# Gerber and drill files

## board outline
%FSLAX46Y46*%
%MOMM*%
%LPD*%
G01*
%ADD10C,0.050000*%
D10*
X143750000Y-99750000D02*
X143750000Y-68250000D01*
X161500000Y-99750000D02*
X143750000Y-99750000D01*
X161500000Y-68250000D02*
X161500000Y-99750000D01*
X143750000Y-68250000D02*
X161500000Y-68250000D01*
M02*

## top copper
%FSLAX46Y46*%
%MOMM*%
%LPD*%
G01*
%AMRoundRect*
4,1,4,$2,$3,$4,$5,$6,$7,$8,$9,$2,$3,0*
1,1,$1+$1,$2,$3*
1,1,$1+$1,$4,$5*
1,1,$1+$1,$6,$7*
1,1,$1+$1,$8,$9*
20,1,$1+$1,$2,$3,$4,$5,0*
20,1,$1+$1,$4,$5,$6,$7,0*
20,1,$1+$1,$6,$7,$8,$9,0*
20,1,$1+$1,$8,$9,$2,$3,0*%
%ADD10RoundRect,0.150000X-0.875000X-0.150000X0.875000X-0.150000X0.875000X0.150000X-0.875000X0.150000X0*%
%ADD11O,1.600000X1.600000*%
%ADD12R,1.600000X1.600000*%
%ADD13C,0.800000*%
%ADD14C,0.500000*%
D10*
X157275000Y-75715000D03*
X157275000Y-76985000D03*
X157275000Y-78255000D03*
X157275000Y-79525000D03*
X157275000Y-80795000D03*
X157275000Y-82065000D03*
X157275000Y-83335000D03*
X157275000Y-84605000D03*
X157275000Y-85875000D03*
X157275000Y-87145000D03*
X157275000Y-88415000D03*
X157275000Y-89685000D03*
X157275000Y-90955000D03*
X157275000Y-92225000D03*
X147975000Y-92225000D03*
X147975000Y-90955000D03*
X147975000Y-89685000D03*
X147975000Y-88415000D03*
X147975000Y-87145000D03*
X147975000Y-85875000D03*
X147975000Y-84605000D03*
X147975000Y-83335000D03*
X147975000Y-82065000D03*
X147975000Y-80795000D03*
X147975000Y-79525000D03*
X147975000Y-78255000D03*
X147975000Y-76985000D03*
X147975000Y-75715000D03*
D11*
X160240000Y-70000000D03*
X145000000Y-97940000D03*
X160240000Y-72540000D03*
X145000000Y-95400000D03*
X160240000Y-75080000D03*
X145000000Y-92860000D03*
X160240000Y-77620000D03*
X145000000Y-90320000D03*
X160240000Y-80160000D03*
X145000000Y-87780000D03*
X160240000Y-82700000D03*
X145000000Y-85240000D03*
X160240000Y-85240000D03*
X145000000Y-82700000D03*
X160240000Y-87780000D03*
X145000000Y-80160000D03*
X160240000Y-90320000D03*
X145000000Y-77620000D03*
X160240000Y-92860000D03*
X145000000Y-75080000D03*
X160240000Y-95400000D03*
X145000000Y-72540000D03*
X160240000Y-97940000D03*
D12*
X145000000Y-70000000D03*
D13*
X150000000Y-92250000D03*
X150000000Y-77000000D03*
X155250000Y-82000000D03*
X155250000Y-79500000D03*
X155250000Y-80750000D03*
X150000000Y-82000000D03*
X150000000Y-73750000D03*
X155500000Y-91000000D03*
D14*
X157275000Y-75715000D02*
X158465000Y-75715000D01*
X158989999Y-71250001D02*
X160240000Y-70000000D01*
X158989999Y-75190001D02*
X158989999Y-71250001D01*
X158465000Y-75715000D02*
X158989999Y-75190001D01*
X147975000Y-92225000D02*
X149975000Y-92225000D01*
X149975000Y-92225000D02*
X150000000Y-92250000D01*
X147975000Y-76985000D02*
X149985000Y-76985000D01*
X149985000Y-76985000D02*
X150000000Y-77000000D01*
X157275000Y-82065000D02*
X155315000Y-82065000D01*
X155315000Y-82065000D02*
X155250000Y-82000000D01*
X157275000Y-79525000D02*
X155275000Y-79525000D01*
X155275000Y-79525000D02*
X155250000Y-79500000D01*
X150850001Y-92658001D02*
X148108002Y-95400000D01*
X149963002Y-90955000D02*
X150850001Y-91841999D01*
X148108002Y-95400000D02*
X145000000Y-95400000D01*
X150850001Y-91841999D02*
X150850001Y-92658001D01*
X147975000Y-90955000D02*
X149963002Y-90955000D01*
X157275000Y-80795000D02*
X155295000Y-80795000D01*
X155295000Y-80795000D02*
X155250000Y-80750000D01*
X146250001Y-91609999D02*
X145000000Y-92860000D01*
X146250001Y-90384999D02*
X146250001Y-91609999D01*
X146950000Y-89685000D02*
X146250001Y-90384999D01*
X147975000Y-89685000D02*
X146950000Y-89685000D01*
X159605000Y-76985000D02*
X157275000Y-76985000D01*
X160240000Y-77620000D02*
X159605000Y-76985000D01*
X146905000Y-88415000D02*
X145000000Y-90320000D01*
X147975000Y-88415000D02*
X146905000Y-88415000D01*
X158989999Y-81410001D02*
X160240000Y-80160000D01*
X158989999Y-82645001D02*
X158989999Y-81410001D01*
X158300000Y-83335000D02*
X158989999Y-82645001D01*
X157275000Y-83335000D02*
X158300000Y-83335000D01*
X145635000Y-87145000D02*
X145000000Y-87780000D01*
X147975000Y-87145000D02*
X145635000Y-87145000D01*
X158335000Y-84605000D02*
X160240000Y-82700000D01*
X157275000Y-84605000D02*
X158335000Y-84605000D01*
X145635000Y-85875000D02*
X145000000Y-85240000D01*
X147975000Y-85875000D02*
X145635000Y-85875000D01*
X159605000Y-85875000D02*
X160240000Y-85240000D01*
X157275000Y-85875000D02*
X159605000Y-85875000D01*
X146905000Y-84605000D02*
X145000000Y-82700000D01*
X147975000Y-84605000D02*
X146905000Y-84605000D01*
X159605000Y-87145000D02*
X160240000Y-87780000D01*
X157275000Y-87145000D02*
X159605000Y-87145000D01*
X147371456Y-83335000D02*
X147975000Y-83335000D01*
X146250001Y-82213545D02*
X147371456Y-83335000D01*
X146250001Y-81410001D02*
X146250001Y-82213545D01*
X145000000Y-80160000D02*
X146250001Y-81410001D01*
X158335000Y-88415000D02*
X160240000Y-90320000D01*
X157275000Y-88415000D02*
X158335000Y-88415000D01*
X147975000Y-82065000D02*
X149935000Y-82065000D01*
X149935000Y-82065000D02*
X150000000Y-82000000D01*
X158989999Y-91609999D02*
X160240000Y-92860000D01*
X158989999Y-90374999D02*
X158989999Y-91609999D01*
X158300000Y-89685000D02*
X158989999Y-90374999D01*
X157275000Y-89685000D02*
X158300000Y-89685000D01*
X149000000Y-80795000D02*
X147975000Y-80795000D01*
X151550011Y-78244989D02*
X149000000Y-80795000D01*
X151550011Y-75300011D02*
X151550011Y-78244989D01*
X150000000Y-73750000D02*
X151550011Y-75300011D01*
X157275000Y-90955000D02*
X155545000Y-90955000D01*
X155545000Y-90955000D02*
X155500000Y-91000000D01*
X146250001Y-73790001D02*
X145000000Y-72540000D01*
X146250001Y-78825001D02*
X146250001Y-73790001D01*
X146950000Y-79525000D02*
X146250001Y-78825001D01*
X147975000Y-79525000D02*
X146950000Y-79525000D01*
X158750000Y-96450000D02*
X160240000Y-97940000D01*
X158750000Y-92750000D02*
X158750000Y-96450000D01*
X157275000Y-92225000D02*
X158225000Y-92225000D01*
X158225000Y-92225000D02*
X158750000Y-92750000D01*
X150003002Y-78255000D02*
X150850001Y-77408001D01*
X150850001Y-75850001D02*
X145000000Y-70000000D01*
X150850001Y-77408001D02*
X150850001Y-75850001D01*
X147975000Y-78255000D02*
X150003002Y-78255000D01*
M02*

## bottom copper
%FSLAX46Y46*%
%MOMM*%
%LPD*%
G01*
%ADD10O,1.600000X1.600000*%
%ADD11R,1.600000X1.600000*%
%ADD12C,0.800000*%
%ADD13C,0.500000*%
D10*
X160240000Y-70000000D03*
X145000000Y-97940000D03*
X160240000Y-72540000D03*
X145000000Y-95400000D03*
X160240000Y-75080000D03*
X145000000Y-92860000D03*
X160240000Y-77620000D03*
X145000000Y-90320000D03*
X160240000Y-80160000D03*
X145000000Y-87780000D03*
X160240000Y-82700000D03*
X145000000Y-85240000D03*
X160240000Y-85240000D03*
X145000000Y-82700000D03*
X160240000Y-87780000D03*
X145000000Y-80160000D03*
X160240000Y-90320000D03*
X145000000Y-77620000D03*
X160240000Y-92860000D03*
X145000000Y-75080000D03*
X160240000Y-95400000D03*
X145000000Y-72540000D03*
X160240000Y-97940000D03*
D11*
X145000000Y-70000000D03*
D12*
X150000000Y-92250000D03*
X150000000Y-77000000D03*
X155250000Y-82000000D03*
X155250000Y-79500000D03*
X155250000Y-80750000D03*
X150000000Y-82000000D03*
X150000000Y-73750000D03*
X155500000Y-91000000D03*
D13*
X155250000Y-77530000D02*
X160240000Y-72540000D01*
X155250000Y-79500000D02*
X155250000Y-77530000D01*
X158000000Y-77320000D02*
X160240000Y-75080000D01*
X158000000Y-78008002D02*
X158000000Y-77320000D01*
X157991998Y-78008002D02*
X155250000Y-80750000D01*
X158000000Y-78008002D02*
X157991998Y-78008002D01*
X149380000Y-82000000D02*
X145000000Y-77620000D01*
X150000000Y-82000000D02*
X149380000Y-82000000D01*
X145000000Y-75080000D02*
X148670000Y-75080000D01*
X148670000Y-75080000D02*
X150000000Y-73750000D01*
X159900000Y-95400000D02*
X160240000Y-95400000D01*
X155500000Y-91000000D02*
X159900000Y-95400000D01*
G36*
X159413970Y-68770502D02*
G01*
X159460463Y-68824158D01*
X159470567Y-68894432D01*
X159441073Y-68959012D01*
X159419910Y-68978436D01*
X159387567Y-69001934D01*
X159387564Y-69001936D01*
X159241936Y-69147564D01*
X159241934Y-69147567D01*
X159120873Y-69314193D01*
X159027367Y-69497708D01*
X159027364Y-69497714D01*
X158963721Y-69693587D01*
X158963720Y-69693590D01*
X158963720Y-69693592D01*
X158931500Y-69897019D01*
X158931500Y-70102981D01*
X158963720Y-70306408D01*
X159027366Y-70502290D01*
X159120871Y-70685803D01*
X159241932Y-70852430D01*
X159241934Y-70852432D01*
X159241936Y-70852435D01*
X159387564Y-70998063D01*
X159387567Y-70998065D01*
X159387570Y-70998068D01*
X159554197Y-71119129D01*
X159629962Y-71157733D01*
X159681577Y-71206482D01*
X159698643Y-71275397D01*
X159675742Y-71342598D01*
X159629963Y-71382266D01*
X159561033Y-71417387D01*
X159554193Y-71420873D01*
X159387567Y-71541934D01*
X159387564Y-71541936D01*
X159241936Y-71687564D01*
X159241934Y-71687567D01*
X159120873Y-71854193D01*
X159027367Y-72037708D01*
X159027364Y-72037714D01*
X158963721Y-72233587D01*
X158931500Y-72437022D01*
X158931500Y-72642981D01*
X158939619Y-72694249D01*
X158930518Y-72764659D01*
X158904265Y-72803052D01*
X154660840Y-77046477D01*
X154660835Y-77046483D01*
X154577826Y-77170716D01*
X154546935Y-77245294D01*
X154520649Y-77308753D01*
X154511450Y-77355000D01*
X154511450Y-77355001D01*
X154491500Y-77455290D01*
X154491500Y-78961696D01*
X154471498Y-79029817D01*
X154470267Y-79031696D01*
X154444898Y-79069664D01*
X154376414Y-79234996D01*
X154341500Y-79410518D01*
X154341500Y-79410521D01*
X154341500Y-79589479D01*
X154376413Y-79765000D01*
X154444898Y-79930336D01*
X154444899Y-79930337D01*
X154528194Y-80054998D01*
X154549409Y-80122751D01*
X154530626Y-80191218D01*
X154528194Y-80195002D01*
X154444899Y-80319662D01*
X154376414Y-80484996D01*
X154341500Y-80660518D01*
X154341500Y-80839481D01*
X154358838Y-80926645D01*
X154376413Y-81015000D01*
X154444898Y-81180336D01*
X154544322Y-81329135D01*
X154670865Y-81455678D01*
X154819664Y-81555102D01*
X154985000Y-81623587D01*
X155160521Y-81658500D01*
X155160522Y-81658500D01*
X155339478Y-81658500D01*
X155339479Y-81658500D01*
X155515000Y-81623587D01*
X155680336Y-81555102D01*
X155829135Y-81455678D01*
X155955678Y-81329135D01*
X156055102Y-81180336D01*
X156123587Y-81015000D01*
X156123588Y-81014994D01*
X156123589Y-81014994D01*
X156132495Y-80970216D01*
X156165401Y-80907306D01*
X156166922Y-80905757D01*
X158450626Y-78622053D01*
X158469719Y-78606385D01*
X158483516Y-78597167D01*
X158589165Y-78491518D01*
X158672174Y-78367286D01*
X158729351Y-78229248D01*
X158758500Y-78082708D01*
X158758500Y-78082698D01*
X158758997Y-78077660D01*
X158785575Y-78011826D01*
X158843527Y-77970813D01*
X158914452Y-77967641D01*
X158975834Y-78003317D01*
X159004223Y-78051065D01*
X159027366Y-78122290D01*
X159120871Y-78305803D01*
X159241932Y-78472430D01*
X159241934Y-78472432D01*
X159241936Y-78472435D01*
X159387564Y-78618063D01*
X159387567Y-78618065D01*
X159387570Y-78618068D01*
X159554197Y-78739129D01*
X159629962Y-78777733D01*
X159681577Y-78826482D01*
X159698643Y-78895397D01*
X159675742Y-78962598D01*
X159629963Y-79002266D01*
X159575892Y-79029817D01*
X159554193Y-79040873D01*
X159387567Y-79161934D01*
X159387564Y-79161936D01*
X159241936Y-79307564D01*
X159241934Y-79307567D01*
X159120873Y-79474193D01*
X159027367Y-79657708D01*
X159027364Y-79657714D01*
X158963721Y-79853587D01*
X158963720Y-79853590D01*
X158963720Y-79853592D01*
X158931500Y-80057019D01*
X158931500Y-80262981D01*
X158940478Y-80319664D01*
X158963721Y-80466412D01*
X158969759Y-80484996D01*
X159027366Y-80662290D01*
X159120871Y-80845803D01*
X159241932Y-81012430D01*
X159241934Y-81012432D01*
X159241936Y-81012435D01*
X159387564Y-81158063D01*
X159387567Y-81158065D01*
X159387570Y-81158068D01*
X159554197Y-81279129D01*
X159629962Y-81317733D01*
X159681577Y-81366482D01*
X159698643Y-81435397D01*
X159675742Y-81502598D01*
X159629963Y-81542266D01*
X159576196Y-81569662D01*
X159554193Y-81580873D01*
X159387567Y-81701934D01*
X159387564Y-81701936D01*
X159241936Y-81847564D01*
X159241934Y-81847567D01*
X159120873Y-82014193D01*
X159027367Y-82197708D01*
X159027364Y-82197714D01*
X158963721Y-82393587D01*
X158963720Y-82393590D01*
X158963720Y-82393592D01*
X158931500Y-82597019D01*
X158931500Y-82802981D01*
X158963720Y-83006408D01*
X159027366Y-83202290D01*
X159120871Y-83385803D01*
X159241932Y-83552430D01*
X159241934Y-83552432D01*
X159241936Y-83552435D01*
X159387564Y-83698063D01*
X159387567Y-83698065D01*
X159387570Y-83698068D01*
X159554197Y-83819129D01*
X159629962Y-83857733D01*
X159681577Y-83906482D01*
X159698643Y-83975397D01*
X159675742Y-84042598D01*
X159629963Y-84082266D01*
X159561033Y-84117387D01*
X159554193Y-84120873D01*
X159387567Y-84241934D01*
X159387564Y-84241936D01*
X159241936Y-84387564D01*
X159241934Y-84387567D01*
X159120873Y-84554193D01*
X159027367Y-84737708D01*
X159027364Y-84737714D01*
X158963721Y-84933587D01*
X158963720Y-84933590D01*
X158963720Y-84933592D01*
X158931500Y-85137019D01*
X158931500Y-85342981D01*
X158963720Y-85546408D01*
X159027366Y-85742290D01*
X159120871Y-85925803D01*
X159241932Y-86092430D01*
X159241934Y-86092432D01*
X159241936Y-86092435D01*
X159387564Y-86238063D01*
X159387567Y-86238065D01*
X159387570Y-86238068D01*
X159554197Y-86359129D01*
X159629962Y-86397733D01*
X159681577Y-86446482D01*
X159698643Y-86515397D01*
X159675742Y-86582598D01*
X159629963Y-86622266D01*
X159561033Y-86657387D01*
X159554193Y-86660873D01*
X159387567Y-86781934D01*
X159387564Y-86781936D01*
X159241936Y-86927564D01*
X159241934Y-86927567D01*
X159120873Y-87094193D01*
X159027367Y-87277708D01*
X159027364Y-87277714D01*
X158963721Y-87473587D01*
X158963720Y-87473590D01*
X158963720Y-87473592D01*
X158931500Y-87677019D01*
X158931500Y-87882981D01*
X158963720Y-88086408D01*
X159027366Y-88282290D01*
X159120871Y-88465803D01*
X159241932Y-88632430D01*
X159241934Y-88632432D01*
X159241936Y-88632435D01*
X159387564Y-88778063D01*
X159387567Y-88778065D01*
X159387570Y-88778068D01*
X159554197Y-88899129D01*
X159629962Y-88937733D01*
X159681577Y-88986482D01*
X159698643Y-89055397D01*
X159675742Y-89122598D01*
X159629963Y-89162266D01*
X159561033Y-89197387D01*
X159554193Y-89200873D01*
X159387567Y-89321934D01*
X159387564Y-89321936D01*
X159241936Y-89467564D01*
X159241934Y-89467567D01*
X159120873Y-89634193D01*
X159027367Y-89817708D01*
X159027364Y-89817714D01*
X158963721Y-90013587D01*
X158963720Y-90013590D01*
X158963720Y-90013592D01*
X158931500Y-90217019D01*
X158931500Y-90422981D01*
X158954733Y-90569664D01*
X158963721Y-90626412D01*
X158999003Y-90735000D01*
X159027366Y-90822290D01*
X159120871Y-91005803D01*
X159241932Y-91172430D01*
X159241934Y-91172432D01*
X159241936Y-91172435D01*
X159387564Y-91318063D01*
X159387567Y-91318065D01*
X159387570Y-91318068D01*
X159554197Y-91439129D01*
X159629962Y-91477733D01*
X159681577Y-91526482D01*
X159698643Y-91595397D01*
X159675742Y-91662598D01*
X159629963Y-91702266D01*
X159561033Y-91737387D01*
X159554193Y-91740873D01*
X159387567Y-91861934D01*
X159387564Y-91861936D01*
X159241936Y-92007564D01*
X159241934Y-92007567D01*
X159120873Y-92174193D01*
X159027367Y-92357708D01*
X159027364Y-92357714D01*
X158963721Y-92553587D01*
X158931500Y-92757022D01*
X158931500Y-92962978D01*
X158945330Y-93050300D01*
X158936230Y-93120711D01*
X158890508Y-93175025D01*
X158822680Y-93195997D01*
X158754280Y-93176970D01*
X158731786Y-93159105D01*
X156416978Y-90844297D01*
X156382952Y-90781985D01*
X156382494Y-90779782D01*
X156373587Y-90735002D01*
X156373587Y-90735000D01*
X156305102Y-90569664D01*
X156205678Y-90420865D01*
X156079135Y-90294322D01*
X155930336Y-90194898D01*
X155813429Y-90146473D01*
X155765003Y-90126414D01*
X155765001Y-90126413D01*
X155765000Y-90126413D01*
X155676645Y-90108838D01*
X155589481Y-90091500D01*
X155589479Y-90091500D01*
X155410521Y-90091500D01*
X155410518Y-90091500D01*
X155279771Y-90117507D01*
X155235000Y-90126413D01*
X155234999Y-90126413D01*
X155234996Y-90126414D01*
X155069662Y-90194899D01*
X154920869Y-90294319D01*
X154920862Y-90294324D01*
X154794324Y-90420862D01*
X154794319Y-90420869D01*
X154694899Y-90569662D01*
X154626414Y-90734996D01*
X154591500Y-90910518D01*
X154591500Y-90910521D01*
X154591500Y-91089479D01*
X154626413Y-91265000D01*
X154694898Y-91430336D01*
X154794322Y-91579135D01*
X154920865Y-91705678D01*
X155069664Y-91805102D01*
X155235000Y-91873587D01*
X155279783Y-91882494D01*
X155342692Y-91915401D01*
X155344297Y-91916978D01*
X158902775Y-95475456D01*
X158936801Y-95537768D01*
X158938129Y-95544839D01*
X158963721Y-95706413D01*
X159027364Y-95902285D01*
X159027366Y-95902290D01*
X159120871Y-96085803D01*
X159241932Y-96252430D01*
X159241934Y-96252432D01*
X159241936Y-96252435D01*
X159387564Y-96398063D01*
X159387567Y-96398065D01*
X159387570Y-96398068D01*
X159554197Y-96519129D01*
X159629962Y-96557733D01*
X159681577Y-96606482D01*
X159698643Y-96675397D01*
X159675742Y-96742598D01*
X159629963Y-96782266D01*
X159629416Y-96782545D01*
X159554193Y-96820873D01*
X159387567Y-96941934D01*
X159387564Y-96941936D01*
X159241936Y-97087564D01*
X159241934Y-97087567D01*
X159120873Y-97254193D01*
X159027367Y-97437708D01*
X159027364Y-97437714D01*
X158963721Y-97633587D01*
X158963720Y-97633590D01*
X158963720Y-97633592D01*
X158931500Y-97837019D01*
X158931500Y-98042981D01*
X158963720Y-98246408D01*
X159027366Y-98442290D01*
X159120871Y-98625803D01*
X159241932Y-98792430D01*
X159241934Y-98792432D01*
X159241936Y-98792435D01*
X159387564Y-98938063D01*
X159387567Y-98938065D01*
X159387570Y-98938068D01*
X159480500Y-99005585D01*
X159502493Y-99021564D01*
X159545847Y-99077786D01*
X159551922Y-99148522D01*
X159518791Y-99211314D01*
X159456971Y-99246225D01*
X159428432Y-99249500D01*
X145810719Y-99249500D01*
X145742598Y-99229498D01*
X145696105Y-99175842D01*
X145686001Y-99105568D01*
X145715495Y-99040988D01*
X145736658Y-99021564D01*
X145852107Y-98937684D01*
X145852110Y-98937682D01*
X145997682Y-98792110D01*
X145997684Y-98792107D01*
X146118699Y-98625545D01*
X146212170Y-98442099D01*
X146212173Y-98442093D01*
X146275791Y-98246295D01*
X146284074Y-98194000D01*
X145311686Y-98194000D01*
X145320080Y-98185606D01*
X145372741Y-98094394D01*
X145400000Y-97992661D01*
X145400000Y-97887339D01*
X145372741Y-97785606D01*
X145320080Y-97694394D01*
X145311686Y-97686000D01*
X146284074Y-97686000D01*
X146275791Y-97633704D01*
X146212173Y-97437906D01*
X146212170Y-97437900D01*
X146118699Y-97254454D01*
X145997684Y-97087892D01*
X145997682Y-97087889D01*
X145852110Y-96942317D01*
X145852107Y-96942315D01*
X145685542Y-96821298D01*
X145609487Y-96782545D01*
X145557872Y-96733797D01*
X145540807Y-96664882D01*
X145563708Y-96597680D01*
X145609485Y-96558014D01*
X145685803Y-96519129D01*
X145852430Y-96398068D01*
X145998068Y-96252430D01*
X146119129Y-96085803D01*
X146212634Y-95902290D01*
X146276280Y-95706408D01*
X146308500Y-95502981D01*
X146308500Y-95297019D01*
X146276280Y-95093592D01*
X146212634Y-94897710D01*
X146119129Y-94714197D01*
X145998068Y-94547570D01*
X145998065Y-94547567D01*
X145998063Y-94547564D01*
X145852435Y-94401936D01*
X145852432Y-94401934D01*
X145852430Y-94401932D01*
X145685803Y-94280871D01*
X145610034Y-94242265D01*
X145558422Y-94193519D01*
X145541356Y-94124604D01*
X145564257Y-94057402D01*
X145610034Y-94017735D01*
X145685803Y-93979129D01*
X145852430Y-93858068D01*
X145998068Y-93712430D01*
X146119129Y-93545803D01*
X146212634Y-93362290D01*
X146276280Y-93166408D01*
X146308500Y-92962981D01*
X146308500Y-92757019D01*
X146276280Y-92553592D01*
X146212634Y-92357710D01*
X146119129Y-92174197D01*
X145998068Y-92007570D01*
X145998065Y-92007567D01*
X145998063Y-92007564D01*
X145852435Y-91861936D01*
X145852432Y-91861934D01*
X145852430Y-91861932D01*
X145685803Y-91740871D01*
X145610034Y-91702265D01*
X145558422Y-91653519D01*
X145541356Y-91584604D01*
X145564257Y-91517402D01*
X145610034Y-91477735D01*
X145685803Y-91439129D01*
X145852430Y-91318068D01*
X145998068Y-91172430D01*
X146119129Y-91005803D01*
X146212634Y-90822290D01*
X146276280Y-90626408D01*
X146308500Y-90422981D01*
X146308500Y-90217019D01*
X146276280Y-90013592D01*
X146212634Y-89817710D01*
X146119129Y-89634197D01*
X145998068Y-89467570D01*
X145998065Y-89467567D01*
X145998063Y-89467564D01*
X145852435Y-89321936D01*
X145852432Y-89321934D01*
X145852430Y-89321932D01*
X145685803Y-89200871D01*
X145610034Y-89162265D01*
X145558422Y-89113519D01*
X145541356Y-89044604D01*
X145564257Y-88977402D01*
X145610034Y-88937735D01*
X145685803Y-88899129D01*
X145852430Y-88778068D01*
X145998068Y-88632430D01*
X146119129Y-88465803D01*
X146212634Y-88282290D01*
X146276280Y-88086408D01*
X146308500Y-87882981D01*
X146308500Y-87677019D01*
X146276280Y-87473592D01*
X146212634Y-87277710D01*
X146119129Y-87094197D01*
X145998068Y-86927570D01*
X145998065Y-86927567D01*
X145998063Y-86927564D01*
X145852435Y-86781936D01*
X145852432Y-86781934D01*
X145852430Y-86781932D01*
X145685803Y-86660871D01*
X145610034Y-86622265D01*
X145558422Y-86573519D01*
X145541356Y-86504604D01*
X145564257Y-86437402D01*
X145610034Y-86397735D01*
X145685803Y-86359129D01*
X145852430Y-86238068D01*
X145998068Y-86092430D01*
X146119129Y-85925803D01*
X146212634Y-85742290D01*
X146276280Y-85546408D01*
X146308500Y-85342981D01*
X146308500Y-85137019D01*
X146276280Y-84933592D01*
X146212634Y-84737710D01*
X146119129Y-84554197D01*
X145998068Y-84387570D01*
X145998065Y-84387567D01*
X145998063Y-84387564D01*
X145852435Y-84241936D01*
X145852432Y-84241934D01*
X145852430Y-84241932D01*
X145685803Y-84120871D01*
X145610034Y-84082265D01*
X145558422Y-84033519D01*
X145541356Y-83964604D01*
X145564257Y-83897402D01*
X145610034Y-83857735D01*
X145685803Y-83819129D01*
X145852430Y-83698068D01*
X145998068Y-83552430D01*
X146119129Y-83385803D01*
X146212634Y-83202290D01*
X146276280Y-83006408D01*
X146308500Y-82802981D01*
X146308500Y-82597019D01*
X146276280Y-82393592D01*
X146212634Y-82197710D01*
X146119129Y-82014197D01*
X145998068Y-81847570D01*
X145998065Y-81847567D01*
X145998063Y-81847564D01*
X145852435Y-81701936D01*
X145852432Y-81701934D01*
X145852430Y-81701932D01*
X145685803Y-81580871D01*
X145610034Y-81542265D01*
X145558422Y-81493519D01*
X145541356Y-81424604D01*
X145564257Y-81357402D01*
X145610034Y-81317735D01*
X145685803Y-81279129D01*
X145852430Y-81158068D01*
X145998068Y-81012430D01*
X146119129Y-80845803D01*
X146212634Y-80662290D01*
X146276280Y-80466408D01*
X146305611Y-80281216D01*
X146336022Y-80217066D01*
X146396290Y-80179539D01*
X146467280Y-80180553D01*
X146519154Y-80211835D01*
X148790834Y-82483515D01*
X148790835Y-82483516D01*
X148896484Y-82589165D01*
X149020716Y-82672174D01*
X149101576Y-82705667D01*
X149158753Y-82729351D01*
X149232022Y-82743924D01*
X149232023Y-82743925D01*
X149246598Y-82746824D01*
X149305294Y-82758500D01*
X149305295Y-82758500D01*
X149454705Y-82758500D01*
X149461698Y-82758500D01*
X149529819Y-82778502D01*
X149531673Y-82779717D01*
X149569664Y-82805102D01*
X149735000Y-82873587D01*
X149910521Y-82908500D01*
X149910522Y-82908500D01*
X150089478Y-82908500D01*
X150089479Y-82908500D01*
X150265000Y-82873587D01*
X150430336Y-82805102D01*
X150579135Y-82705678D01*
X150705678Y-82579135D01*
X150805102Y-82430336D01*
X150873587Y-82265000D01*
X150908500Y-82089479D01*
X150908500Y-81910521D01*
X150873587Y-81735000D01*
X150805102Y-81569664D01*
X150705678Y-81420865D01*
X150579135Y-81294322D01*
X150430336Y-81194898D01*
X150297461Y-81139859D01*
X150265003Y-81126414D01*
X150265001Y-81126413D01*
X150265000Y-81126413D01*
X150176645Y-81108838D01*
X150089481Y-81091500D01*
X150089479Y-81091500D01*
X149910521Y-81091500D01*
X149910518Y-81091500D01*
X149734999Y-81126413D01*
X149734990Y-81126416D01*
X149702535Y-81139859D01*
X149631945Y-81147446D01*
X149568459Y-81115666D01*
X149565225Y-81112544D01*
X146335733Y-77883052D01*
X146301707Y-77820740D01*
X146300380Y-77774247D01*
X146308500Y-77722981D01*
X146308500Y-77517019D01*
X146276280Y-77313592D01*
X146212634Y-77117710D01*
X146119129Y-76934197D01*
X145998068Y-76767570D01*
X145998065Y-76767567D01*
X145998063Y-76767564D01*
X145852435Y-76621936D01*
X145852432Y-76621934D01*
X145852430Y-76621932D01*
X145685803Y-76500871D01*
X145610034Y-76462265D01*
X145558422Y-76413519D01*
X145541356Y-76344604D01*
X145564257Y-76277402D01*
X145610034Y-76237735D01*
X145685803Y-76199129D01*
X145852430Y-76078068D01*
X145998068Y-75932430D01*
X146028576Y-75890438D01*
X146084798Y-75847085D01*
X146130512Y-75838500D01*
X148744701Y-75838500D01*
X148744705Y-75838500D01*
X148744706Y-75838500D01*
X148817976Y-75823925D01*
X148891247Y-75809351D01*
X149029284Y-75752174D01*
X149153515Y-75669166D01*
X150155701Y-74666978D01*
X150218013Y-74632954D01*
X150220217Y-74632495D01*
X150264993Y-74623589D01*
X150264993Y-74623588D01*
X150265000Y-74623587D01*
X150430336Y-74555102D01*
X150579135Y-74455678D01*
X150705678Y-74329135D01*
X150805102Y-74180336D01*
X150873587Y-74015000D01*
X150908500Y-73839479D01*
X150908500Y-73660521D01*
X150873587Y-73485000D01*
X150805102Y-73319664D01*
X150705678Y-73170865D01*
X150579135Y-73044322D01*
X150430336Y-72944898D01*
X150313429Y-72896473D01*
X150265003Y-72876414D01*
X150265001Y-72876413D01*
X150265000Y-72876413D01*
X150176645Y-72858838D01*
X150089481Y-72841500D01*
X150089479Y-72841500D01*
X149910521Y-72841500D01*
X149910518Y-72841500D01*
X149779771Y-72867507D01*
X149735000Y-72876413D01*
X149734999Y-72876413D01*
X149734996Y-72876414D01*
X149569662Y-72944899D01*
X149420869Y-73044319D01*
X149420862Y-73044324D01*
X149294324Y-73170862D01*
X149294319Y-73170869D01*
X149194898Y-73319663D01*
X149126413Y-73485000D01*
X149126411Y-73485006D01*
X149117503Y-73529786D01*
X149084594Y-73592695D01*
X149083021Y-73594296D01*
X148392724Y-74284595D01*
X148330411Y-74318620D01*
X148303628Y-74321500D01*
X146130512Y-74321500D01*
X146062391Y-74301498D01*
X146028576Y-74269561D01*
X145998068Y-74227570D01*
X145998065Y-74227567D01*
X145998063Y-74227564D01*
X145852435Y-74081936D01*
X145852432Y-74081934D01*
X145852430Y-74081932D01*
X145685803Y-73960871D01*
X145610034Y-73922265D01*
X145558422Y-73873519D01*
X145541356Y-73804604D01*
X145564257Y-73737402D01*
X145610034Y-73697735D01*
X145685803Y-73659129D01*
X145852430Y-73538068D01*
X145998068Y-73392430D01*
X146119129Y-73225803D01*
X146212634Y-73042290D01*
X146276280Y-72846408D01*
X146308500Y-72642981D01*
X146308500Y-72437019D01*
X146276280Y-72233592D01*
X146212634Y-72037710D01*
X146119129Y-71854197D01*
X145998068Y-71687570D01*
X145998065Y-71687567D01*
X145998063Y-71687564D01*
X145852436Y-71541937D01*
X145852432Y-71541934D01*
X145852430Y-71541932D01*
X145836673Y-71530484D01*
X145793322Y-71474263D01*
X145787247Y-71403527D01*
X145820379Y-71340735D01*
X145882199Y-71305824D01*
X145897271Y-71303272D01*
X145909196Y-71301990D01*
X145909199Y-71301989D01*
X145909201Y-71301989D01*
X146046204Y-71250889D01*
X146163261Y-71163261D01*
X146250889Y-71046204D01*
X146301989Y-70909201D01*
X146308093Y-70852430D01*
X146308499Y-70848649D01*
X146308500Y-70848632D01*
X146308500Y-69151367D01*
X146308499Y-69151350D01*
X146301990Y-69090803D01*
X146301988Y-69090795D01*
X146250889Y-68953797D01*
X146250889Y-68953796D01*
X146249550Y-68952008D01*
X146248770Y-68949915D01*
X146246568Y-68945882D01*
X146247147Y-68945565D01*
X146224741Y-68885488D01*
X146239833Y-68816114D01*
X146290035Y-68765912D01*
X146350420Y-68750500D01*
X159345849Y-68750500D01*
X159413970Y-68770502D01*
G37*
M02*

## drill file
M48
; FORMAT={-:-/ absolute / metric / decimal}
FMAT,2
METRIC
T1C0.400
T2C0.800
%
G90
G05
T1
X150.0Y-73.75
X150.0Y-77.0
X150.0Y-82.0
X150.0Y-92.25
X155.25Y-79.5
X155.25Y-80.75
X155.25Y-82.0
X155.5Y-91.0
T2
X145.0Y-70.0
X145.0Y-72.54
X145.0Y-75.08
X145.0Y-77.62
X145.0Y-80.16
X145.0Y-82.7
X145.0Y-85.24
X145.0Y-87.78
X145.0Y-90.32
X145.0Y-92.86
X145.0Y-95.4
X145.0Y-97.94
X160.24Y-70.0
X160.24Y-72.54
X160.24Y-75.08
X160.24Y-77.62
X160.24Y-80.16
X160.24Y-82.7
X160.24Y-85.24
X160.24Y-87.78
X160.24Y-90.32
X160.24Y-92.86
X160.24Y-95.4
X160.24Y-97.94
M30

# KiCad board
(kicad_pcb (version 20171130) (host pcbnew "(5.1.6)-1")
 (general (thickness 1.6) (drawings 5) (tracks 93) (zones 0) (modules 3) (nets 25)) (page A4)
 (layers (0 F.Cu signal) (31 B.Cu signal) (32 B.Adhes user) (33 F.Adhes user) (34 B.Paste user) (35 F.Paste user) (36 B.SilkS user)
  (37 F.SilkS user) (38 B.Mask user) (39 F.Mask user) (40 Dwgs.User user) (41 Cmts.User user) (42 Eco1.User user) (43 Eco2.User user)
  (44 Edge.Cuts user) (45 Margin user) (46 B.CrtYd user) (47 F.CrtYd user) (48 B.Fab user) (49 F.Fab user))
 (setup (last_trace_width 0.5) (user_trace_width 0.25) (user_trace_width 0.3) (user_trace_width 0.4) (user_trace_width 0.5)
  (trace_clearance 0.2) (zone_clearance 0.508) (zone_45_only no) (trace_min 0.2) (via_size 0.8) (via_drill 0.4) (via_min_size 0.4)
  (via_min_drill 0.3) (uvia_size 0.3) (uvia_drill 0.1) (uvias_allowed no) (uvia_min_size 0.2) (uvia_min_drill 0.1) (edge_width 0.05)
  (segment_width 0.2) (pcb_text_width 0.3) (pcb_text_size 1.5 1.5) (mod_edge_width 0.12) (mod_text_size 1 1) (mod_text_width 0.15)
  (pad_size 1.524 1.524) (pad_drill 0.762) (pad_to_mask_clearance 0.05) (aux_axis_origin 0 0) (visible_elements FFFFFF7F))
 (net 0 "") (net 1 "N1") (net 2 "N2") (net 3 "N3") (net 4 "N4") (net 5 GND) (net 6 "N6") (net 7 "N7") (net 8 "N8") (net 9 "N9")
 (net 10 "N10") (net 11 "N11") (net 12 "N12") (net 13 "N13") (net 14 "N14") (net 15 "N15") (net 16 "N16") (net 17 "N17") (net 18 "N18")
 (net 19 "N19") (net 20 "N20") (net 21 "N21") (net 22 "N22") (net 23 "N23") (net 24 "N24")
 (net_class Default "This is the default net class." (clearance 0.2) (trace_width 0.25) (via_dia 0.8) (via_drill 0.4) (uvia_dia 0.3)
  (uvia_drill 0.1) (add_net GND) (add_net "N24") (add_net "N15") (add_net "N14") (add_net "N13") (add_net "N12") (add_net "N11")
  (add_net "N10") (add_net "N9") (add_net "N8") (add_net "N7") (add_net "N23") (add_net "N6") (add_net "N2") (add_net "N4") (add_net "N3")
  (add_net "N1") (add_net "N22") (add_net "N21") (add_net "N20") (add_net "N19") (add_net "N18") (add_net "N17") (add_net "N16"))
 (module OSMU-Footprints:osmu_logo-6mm (layer F.Cu) (at 152.625 72)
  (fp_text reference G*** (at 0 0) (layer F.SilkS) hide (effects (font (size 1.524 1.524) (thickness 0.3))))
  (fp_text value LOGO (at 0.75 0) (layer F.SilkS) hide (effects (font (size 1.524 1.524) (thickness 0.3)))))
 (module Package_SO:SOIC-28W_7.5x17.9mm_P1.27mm (layer F.Cu) (at 152.625 83.97)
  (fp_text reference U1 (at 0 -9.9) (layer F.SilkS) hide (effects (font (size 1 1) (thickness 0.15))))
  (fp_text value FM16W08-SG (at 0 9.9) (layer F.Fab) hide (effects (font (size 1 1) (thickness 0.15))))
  (pad 28 smd roundrect (at 4.65 -8.255) (size 2.05 0.6) (layers F.Cu F.Paste F.Mask) (roundrect_rratio 0.25) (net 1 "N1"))
  (pad 27 smd roundrect (at 4.65 -6.985) (size 2.05 0.6) (layers F.Cu F.Paste F.Mask) (roundrect_rratio 0.25) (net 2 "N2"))
  (pad 26 smd roundrect (at 4.65 -5.715) (size 2.05 0.6) (layers F.Cu F.Paste F.Mask) (roundrect_rratio 0.25))
  (pad 25 smd roundrect (at 4.65 -4.445) (size 2.05 0.6) (layers F.Cu F.Paste F.Mask) (roundrect_rratio 0.25) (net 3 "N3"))
  (pad 24 smd roundrect (at 4.65 -3.175) (size 2.05 0.6) (layers F.Cu F.Paste F.Mask) (roundrect_rratio 0.25) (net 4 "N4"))
  (pad 23 smd roundrect (at 4.65 -1.905) (size 2.05 0.6) (layers F.Cu F.Paste F.Mask) (roundrect_rratio 0.25) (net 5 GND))
  (pad 22 smd roundrect (at 4.65 -0.635) (size 2.05 0.6) (layers F.Cu F.Paste F.Mask) (roundrect_rratio 0.25) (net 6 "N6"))
  (pad 21 smd roundrect (at 4.65 0.635) (size 2.05 0.6) (layers F.Cu F.Paste F.Mask) (roundrect_rratio 0.25) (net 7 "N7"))
  (pad 20 smd roundrect (at 4.65 1.905) (size 2.05 0.6) (layers F.Cu F.Paste F.Mask) (roundrect_rratio 0.25) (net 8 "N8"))
  (pad 19 smd roundrect (at 4.65 3.175) (size 2.05 0.6) (layers F.Cu F.Paste F.Mask) (roundrect_rratio 0.25) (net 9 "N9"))
  (pad 18 smd roundrect (at 4.65 4.445) (size 2.05 0.6) (layers F.Cu F.Paste F.Mask) (roundrect_rratio 0.25) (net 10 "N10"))
  (pad 17 smd roundrect (at 4.65 5.715) (size 2.05 0.6) (layers F.Cu F.Paste F.Mask) (roundrect_rratio 0.25) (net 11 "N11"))
  (pad 16 smd roundrect (at 4.65 6.985) (size 2.05 0.6) (layers F.Cu F.Paste F.Mask) (roundrect_rratio 0.25) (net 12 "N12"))
  (pad 15 smd roundrect (at 4.65 8.255) (size 2.05 0.6) (layers F.Cu F.Paste F.Mask) (roundrect_rratio 0.25) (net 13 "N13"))
  (pad 14 smd roundrect (at -4.65 8.255) (size 2.05 0.6) (layers F.Cu F.Paste F.Mask) (roundrect_rratio 0.25) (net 5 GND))
  (pad 13 smd roundrect (at -4.65 6.985) (size 2.05 0.6) (layers F.Cu F.Paste F.Mask) (roundrect_rratio 0.25) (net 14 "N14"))
  (pad 12 smd roundrect (at -4.65 5.715) (size 2.05 0.6) (layers F.Cu F.Paste F.Mask) (roundrect_rratio 0.25) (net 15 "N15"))
  (pad 11 smd roundrect (at -4.65 4.445) (size 2.05 0.6) (layers F.Cu F.Paste F.Mask) (roundrect_rratio 0.25) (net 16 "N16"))
  (pad 10 smd roundrect (at -4.65 3.175) (size 2.05 0.6) (layers F.Cu F.Paste F.Mask) (roundrect_rratio 0.25) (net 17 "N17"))
  (pad 9 smd roundrect (at -4.65 1.905) (size 2.05 0.6) (layers F.Cu F.Paste F.Mask) (roundrect_rratio 0.25) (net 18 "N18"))
  (pad 8 smd roundrect (at -4.65 0.635) (size 2.05 0.6) (layers F.Cu F.Paste F.Mask) (roundrect_rratio 0.25) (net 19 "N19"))
  (pad 7 smd roundrect (at -4.65 -0.635) (size 2.05 0.6) (layers F.Cu F.Paste F.Mask) (roundrect_rratio 0.25) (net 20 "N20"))
  (pad 6 smd roundrect (at -4.65 -1.905) (size 2.05 0.6) (layers F.Cu F.Paste F.Mask) (roundrect_rratio 0.25) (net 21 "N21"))
  (pad 5 smd roundrect (at -4.65 -3.175) (size 2.05 0.6) (layers F.Cu F.Paste F.Mask) (roundrect_rratio 0.25) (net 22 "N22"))
  (pad 4 smd roundrect (at -4.65 -4.445) (size 2.05 0.6) (layers F.Cu F.Paste F.Mask) (roundrect_rratio 0.25) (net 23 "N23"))
  (pad 3 smd roundrect (at -4.65 -5.715) (size 2.05 0.6) (layers F.Cu F.Paste F.Mask) (roundrect_rratio 0.25) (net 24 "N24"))
  (pad 2 smd roundrect (at -4.65 -6.985) (size 2.05 0.6) (layers F.Cu F.Paste F.Mask) (roundrect_rratio 0.25) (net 5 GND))
  (pad 1 smd roundrect (at -4.65 -8.255) (size 2.05 0.6) (layers F.Cu F.Paste F.Mask) (roundrect_rratio 0.25)))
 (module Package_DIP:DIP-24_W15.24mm (layer F.Cu) (at 145 70)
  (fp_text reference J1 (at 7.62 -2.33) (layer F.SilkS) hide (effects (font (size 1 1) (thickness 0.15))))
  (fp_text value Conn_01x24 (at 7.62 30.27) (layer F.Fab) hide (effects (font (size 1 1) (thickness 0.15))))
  (pad 24 thru_hole oval (at 15.24 0) (size 1.6 1.6) (drill 0.8) (layers *.Cu *.Mask) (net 1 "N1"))
  (pad 12 thru_hole oval (at 0 27.94) (size 1.6 1.6) (drill 0.8) (layers *.Cu *.Mask) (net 5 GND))
  (pad 23 thru_hole oval (at 15.24 2.54) (size 1.6 1.6) (drill 0.8) (layers *.Cu *.Mask) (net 3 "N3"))
  (pad 11 thru_hole oval (at 0 25.4) (size 1.6 1.6) (drill 0.8) (layers *.Cu *.Mask) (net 14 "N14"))
  (pad 22 thru_hole oval (at 15.24 5.08) (size 1.6 1.6) (drill 0.8) (layers *.Cu *.Mask) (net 4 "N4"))
  (pad 10 thru_hole oval (at 0 22.86) (size 1.6 1.6) (drill 0.8) (layers *.Cu *.Mask) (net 15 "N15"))
  (pad 21 thru_hole oval (at 15.24 7.62) (size 1.6 1.6) (drill 0.8) (layers *.Cu *.Mask) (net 2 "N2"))
  (pad 9 thru_hole oval (at 0 20.32) (size 1.6 1.6) (drill 0.8) (layers *.Cu *.Mask) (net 16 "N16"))
  (pad 20 thru_hole oval (at 15.24 10.16) (size 1.6 1.6) (drill 0.8) (layers *.Cu *.Mask) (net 6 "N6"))
  (pad 8 thru_hole oval (at 0 17.78) (size 1.6 1.6) (drill 0.8) (layers *.Cu *.Mask) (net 17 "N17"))
  (pad 19 thru_hole oval (at 15.24 12.7) (size 1.6 1.6) (drill 0.8) (layers *.Cu *.Mask) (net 7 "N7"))
  (pad 7 thru_hole oval (at 0 15.24) (size 1.6 1.6) (drill 0.8) (layers *.Cu *.Mask) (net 18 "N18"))
  (pad 18 thru_hole oval (at 15.24 15.24) (size 1.6 1.6) (drill 0.8) (layers *.Cu *.Mask) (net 8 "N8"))
  (pad 6 thru_hole oval (at 0 12.7) (size 1.6 1.6) (drill 0.8) (layers *.Cu *.Mask) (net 19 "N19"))
  (pad 17 thru_hole oval (at 15.24 17.78) (size 1.6 1.6) (drill 0.8) (layers *.Cu *.Mask) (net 9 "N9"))
  (pad 5 thru_hole oval (at 0 10.16) (size 1.6 1.6) (drill 0.8) (layers *.Cu *.Mask) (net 20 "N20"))
  (pad 16 thru_hole oval (at 15.24 20.32) (size 1.6 1.6) (drill 0.8) (layers *.Cu *.Mask) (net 10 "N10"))
  (pad 4 thru_hole oval (at 0 7.62) (size 1.6 1.6) (drill 0.8) (layers *.Cu *.Mask) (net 21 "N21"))
  (pad 15 thru_hole oval (at 15.24 22.86) (size 1.6 1.6) (drill 0.8) (layers *.Cu *.Mask) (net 11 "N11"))
  (pad 3 thru_hole oval (at 0 5.08) (size 1.6 1.6) (drill 0.8) (layers *.Cu *.Mask) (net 22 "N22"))
  (pad 14 thru_hole oval (at 15.24 25.4) (size 1.6 1.6) (drill 0.8) (layers *.Cu *.Mask) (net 12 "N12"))
  (pad 2 thru_hole oval (at 0 2.54) (size 1.6 1.6) (drill 0.8) (layers *.Cu *.Mask) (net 23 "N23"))
  (pad 13 thru_hole oval (at 15.24 27.94) (size 1.6 1.6) (drill 0.8) (layers *.Cu *.Mask) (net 13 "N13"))
  (pad 1 thru_hole rect (at 0 0) (size 1.6 1.6) (drill 0.8) (layers *.Cu *.Mask) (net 24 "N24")))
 (gr_line (start 143.75 99.75) (end 143.75 68.25) (layer Edge.Cuts) (width 0.05))
 (gr_line (start 161.5 99.75) (end 143.75 99.75) (layer Edge.Cuts) (width 0.05))
 (gr_line (start 161.5 68.25) (end 161.5 99.75) (layer Edge.Cuts) (width 0.05))
 (gr_line (start 143.75 68.25) (end 161.5 68.25) (layer Edge.Cuts) (width 0.05))
 (segment (start 157.275 75.715) (end 158.465 75.715) (width 0.5) (layer F.Cu) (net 1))
 (segment (start 158.989999 71.250001) (end 160.24 70) (width 0.5) (layer F.Cu) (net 1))
 (segment (start 158.989999 75.190001) (end 158.989999 71.250001) (width 0.5) (layer F.Cu) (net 1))
 (segment (start 158.465 75.715) (end 158.989999 75.190001) (width 0.5) (layer F.Cu) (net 1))
 (via (at 150 92.25) (size 0.8) (drill 0.4) (layers F.Cu B.Cu) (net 5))
 (segment (start 147.975 92.225) (end 149.975 92.225) (width 0.5) (layer F.Cu) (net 5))
 (segment (start 149.975 92.225) (end 150 92.25) (width 0.5) (layer F.Cu) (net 5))
 (via (at 150 77) (size 0.8) (drill 0.4) (layers F.Cu B.Cu) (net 5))
 (segment (start 147.975 76.985) (end 149.985 76.985) (width 0.5) (layer F.Cu) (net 5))
 (segment (start 149.985 76.985) (end 150 77) (width 0.5) (layer F.Cu) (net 5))
 (via (at 155.25 82) (size 0.8) (drill 0.4) (layers F.Cu B.Cu) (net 5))
 (segment (start 157.275 82.065) (end 155.315 82.065) (width 0.5) (layer F.Cu) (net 5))
 (segment (start 155.315 82.065) (end 155.25 82) (width 0.5) (layer F.Cu) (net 5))
 (via (at 155.25 79.5) (size 0.8) (drill 0.4) (layers F.Cu B.Cu) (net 3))
 (segment (start 157.275 79.525) (end 155.275 79.525) (width 0.5) (layer F.Cu) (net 3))
 (segment (start 155.275 79.525) (end 155.25 79.5) (width 0.5) (layer F.Cu) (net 3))
 (segment (start 155.25 77.53) (end 160.24 72.54) (width 0.5) (layer B.Cu) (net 3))
 (segment (start 155.25 79.5) (end 155.25 77.53) (width 0.5) (layer B.Cu) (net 3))
 (segment (start 150.850001 92.658001) (end 148.108002 95.4) (width 0.5) (layer F.Cu) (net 14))
 (segment (start 149.963002 90.955) (end 150.850001 91.841999) (width 0.5) (layer F.Cu) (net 14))
 (segment (start 148.108002 95.4) (end 145 95.4) (width 0.5) (layer F.Cu) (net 14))
 (segment (start 150.850001 91.841999) (end 150.850001 92.658001) (width 0.5) (layer F.Cu) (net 14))
 (segment (start 147.975 90.955) (end 149.963002 90.955) (width 0.5) (layer F.Cu) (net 14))
 (via (at 155.25 80.75) (size 0.8) (drill 0.4) (layers F.Cu B.Cu) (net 4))
 (segment (start 157.275 80.795) (end 155.295 80.795) (width 0.5) (layer F.Cu) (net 4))
 (segment (start 155.295 80.795) (end 155.25 80.75) (width 0.5) (layer F.Cu) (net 4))
 (segment (start 158 77.32) (end 160.24 75.08) (width 0.5) (layer B.Cu) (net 4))
 (segment (start 158 78.008002) (end 158 77.32) (width 0.5) (layer B.Cu) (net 4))
 (segment (start 157.991998 78.008002) (end 155.25 80.75) (width 0.5) (layer B.Cu) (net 4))
 (segment (start 158 78.008002) (end 157.991998 78.008002) (width 0.5) (layer B.Cu) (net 4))
 (segment (start 146.250001 91.609999) (end 145 92.86) (width 0.5) (layer F.Cu) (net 15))
 (segment (start 146.250001 90.384999) (end 146.250001 91.609999) (width 0.5) (layer F.Cu) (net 15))
 (segment (start 146.95 89.685) (end 146.250001 90.384999) (width 0.5) (layer F.Cu) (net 15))
 (segment (start 147.975 89.685) (end 146.95 89.685) (width 0.5) (layer F.Cu) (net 15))
 (segment (start 159.605 76.985) (end 157.275 76.985) (width 0.5) (layer F.Cu) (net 2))
 (segment (start 160.24 77.62) (end 159.605 76.985) (width 0.5) (layer F.Cu) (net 2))
 (segment (start 146.905 88.415) (end 145 90.32) (width 0.5) (layer F.Cu) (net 16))
 (segment (start 147.975 88.415) (end 146.905 88.415) (width 0.5) (layer F.Cu) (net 16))
 (segment (start 158.989999 81.410001) (end 160.24 80.16) (width 0.5) (layer F.Cu) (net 6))
 (segment (start 158.989999 82.645001) (end 158.989999 81.410001) (width 0.5) (layer F.Cu) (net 6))
 (segment (start 158.3 83.335) (end 158.989999 82.645001) (width 0.5) (layer F.Cu) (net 6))
 (segment (start 157.275 83.335) (end 158.3 83.335) (width 0.5) (layer F.Cu) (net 6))
 (segment (start 145.635 87.145) (end 145 87.78) (width 0.5) (layer F.Cu) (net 17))
 (segment (start 147.975 87.145) (end 145.635 87.145) (width 0.5) (layer F.Cu) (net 17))
 (segment (start 158.335 84.605) (end 160.24 82.7) (width 0.5) (layer F.Cu) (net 7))
 (segment (start 157.275 84.605) (end 158.335 84.605) (width 0.5) (layer F.Cu) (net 7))
 (segment (start 145.635 85.875) (end 145 85.24) (width 0.5) (layer F.Cu) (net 18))
 (segment (start 147.975 85.875) (end 145.635 85.875) (width 0.5) (layer F.Cu) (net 18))
 (segment (start 159.605 85.875) (end 160.24 85.24) (width 0.5) (layer F.Cu) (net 8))
 (segment (start 157.275 85.875) (end 159.605 85.875) (width 0.5) (layer F.Cu) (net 8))
 (segment (start 146.905 84.605) (end 145 82.7) (width 0.5) (layer F.Cu) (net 19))
 (segment (start 147.975 84.605) (end 146.905 84.605) (width 0.5) (layer F.Cu) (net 19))
 (segment (start 159.605 87.145) (end 160.24 87.78) (width 0.5) (layer F.Cu) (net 9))
 (segment (start 157.275 87.145) (end 159.605 87.145) (width 0.5) (layer F.Cu) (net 9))
 (segment (start 147.371456 83.335) (end 147.975 83.335) (width 0.5) (layer F.Cu) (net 20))
 (segment (start 146.250001 82.213545) (end 147.371456 83.335) (width 0.5) (layer F.Cu) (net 20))
 (segment (start 146.250001 81.410001) (end 146.250001 82.213545) (width 0.5) (layer F.Cu) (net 20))
 (segment (start 145 80.16) (end 146.250001 81.410001) (width 0.5) (layer F.Cu) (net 20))
 (segment (start 158.335 88.415) (end 160.24 90.32) (width 0.5) (layer F.Cu) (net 10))
 (segment (start 157.275 88.415) (end 158.335 88.415) (width 0.5) (layer F.Cu) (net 10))
 (via (at 150 82) (size 0.8) (drill 0.4) (layers F.Cu B.Cu) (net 21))
 (segment (start 147.975 82.065) (end 149.935 82.065) (width 0.5) (layer F.Cu) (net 21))
 (segment (start 149.935 82.065) (end 150 82) (width 0.5) (layer F.Cu) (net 21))
 (segment (start 149.38 82) (end 145 77.62) (width 0.5) (layer B.Cu) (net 21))
 (segment (start 150 82) (end 149.38 82) (width 0.5) (layer B.Cu) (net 21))
 (segment (start 158.989999 91.609999) (end 160.24 92.86) (width 0.5) (layer F.Cu) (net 11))
 (segment (start 158.989999 90.374999) (end 158.989999 91.609999) (width 0.5) (layer F.Cu) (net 11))
 (segment (start 158.3 89.685) (end 158.989999 90.374999) (width 0.5) (layer F.Cu) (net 11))
 (segment (start 157.275 89.685) (end 158.3 89.685) (width 0.5) (layer F.Cu) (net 11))
 (via (at 150 73.75) (size 0.8) (drill 0.4) (layers F.Cu B.Cu) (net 22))
 (segment (start 145 75.08) (end 148.67 75.08) (width 0.5) (layer B.Cu) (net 22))
 (segment (start 148.67 75.08) (end 150 73.75) (width 0.5) (layer B.Cu) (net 22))
 (segment (start 149 80.795) (end 147.975 80.795) (width 0.5) (layer F.Cu) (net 22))
 (segment (start 151.550011 78.244989) (end 149 80.795) (width 0.5) (layer F.Cu) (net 22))
 (segment (start 151.550011 75.300011) (end 151.550011 78.244989) (width 0.5) (layer F.Cu) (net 22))
 (segment (start 150 73.75) (end 151.550011 75.300011) (width 0.5) (layer F.Cu) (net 22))
 (via (at 155.5 91) (size 0.8) (drill 0.4) (layers F.Cu B.Cu) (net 12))
 (segment (start 157.275 90.955) (end 155.545 90.955) (width 0.5) (layer F.Cu) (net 12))
 (segment (start 155.545 90.955) (end 155.5 91) (width 0.5) (layer F.Cu) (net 12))
 (segment (start 159.9 95.4) (end 160.24 95.4) (width 0.5) (layer B.Cu) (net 12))
 (segment (start 155.5 91) (end 159.9 95.4) (width 0.5) (layer B.Cu) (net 12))
 (segment (start 146.250001 73.790001) (end 145 72.54) (width 0.5) (layer F.Cu) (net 23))
 (segment (start 146.250001 78.825001) (end 146.250001 73.790001) (width 0.5) (layer F.Cu) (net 23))
 (segment (start 146.95 79.525) (end 146.250001 78.825001) (width 0.5) (layer F.Cu) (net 23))
 (segment (start 147.975 79.525) (end 146.95 79.525) (width 0.5) (layer F.Cu) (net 23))
 (segment (start 158.75 96.45) (end 160.24 97.94) (width 0.5) (layer F.Cu) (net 13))
 (segment (start 158.75 92.75) (end 158.75 96.45) (width 0.5) (layer F.Cu) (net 13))
 (segment (start 157.275 92.225) (end 158.225 92.225) (width 0.5) (layer F.Cu) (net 13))
 (segment (start 158.225 92.225) (end 158.75 92.75) (width 0.5) (layer F.Cu) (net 13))
 (segment (start 150.003002 78.255) (end 150.850001 77.408001) (width 0.5) (layer F.Cu) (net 24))
 (segment (start 150.850001 75.850001) (end 145 70) (width 0.5) (layer F.Cu) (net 24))
 (segment (start 150.850001 77.408001) (end 150.850001 75.850001) (width 0.5) (layer F.Cu) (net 24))
 (segment (start 147.975 78.255) (end 150.003002 78.255) (width 0.5) (layer F.Cu) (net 24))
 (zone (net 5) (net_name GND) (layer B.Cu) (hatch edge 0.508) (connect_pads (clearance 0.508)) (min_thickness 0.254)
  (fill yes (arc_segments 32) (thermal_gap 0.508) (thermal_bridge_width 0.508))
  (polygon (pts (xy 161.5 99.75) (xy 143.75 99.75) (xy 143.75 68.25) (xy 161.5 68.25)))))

